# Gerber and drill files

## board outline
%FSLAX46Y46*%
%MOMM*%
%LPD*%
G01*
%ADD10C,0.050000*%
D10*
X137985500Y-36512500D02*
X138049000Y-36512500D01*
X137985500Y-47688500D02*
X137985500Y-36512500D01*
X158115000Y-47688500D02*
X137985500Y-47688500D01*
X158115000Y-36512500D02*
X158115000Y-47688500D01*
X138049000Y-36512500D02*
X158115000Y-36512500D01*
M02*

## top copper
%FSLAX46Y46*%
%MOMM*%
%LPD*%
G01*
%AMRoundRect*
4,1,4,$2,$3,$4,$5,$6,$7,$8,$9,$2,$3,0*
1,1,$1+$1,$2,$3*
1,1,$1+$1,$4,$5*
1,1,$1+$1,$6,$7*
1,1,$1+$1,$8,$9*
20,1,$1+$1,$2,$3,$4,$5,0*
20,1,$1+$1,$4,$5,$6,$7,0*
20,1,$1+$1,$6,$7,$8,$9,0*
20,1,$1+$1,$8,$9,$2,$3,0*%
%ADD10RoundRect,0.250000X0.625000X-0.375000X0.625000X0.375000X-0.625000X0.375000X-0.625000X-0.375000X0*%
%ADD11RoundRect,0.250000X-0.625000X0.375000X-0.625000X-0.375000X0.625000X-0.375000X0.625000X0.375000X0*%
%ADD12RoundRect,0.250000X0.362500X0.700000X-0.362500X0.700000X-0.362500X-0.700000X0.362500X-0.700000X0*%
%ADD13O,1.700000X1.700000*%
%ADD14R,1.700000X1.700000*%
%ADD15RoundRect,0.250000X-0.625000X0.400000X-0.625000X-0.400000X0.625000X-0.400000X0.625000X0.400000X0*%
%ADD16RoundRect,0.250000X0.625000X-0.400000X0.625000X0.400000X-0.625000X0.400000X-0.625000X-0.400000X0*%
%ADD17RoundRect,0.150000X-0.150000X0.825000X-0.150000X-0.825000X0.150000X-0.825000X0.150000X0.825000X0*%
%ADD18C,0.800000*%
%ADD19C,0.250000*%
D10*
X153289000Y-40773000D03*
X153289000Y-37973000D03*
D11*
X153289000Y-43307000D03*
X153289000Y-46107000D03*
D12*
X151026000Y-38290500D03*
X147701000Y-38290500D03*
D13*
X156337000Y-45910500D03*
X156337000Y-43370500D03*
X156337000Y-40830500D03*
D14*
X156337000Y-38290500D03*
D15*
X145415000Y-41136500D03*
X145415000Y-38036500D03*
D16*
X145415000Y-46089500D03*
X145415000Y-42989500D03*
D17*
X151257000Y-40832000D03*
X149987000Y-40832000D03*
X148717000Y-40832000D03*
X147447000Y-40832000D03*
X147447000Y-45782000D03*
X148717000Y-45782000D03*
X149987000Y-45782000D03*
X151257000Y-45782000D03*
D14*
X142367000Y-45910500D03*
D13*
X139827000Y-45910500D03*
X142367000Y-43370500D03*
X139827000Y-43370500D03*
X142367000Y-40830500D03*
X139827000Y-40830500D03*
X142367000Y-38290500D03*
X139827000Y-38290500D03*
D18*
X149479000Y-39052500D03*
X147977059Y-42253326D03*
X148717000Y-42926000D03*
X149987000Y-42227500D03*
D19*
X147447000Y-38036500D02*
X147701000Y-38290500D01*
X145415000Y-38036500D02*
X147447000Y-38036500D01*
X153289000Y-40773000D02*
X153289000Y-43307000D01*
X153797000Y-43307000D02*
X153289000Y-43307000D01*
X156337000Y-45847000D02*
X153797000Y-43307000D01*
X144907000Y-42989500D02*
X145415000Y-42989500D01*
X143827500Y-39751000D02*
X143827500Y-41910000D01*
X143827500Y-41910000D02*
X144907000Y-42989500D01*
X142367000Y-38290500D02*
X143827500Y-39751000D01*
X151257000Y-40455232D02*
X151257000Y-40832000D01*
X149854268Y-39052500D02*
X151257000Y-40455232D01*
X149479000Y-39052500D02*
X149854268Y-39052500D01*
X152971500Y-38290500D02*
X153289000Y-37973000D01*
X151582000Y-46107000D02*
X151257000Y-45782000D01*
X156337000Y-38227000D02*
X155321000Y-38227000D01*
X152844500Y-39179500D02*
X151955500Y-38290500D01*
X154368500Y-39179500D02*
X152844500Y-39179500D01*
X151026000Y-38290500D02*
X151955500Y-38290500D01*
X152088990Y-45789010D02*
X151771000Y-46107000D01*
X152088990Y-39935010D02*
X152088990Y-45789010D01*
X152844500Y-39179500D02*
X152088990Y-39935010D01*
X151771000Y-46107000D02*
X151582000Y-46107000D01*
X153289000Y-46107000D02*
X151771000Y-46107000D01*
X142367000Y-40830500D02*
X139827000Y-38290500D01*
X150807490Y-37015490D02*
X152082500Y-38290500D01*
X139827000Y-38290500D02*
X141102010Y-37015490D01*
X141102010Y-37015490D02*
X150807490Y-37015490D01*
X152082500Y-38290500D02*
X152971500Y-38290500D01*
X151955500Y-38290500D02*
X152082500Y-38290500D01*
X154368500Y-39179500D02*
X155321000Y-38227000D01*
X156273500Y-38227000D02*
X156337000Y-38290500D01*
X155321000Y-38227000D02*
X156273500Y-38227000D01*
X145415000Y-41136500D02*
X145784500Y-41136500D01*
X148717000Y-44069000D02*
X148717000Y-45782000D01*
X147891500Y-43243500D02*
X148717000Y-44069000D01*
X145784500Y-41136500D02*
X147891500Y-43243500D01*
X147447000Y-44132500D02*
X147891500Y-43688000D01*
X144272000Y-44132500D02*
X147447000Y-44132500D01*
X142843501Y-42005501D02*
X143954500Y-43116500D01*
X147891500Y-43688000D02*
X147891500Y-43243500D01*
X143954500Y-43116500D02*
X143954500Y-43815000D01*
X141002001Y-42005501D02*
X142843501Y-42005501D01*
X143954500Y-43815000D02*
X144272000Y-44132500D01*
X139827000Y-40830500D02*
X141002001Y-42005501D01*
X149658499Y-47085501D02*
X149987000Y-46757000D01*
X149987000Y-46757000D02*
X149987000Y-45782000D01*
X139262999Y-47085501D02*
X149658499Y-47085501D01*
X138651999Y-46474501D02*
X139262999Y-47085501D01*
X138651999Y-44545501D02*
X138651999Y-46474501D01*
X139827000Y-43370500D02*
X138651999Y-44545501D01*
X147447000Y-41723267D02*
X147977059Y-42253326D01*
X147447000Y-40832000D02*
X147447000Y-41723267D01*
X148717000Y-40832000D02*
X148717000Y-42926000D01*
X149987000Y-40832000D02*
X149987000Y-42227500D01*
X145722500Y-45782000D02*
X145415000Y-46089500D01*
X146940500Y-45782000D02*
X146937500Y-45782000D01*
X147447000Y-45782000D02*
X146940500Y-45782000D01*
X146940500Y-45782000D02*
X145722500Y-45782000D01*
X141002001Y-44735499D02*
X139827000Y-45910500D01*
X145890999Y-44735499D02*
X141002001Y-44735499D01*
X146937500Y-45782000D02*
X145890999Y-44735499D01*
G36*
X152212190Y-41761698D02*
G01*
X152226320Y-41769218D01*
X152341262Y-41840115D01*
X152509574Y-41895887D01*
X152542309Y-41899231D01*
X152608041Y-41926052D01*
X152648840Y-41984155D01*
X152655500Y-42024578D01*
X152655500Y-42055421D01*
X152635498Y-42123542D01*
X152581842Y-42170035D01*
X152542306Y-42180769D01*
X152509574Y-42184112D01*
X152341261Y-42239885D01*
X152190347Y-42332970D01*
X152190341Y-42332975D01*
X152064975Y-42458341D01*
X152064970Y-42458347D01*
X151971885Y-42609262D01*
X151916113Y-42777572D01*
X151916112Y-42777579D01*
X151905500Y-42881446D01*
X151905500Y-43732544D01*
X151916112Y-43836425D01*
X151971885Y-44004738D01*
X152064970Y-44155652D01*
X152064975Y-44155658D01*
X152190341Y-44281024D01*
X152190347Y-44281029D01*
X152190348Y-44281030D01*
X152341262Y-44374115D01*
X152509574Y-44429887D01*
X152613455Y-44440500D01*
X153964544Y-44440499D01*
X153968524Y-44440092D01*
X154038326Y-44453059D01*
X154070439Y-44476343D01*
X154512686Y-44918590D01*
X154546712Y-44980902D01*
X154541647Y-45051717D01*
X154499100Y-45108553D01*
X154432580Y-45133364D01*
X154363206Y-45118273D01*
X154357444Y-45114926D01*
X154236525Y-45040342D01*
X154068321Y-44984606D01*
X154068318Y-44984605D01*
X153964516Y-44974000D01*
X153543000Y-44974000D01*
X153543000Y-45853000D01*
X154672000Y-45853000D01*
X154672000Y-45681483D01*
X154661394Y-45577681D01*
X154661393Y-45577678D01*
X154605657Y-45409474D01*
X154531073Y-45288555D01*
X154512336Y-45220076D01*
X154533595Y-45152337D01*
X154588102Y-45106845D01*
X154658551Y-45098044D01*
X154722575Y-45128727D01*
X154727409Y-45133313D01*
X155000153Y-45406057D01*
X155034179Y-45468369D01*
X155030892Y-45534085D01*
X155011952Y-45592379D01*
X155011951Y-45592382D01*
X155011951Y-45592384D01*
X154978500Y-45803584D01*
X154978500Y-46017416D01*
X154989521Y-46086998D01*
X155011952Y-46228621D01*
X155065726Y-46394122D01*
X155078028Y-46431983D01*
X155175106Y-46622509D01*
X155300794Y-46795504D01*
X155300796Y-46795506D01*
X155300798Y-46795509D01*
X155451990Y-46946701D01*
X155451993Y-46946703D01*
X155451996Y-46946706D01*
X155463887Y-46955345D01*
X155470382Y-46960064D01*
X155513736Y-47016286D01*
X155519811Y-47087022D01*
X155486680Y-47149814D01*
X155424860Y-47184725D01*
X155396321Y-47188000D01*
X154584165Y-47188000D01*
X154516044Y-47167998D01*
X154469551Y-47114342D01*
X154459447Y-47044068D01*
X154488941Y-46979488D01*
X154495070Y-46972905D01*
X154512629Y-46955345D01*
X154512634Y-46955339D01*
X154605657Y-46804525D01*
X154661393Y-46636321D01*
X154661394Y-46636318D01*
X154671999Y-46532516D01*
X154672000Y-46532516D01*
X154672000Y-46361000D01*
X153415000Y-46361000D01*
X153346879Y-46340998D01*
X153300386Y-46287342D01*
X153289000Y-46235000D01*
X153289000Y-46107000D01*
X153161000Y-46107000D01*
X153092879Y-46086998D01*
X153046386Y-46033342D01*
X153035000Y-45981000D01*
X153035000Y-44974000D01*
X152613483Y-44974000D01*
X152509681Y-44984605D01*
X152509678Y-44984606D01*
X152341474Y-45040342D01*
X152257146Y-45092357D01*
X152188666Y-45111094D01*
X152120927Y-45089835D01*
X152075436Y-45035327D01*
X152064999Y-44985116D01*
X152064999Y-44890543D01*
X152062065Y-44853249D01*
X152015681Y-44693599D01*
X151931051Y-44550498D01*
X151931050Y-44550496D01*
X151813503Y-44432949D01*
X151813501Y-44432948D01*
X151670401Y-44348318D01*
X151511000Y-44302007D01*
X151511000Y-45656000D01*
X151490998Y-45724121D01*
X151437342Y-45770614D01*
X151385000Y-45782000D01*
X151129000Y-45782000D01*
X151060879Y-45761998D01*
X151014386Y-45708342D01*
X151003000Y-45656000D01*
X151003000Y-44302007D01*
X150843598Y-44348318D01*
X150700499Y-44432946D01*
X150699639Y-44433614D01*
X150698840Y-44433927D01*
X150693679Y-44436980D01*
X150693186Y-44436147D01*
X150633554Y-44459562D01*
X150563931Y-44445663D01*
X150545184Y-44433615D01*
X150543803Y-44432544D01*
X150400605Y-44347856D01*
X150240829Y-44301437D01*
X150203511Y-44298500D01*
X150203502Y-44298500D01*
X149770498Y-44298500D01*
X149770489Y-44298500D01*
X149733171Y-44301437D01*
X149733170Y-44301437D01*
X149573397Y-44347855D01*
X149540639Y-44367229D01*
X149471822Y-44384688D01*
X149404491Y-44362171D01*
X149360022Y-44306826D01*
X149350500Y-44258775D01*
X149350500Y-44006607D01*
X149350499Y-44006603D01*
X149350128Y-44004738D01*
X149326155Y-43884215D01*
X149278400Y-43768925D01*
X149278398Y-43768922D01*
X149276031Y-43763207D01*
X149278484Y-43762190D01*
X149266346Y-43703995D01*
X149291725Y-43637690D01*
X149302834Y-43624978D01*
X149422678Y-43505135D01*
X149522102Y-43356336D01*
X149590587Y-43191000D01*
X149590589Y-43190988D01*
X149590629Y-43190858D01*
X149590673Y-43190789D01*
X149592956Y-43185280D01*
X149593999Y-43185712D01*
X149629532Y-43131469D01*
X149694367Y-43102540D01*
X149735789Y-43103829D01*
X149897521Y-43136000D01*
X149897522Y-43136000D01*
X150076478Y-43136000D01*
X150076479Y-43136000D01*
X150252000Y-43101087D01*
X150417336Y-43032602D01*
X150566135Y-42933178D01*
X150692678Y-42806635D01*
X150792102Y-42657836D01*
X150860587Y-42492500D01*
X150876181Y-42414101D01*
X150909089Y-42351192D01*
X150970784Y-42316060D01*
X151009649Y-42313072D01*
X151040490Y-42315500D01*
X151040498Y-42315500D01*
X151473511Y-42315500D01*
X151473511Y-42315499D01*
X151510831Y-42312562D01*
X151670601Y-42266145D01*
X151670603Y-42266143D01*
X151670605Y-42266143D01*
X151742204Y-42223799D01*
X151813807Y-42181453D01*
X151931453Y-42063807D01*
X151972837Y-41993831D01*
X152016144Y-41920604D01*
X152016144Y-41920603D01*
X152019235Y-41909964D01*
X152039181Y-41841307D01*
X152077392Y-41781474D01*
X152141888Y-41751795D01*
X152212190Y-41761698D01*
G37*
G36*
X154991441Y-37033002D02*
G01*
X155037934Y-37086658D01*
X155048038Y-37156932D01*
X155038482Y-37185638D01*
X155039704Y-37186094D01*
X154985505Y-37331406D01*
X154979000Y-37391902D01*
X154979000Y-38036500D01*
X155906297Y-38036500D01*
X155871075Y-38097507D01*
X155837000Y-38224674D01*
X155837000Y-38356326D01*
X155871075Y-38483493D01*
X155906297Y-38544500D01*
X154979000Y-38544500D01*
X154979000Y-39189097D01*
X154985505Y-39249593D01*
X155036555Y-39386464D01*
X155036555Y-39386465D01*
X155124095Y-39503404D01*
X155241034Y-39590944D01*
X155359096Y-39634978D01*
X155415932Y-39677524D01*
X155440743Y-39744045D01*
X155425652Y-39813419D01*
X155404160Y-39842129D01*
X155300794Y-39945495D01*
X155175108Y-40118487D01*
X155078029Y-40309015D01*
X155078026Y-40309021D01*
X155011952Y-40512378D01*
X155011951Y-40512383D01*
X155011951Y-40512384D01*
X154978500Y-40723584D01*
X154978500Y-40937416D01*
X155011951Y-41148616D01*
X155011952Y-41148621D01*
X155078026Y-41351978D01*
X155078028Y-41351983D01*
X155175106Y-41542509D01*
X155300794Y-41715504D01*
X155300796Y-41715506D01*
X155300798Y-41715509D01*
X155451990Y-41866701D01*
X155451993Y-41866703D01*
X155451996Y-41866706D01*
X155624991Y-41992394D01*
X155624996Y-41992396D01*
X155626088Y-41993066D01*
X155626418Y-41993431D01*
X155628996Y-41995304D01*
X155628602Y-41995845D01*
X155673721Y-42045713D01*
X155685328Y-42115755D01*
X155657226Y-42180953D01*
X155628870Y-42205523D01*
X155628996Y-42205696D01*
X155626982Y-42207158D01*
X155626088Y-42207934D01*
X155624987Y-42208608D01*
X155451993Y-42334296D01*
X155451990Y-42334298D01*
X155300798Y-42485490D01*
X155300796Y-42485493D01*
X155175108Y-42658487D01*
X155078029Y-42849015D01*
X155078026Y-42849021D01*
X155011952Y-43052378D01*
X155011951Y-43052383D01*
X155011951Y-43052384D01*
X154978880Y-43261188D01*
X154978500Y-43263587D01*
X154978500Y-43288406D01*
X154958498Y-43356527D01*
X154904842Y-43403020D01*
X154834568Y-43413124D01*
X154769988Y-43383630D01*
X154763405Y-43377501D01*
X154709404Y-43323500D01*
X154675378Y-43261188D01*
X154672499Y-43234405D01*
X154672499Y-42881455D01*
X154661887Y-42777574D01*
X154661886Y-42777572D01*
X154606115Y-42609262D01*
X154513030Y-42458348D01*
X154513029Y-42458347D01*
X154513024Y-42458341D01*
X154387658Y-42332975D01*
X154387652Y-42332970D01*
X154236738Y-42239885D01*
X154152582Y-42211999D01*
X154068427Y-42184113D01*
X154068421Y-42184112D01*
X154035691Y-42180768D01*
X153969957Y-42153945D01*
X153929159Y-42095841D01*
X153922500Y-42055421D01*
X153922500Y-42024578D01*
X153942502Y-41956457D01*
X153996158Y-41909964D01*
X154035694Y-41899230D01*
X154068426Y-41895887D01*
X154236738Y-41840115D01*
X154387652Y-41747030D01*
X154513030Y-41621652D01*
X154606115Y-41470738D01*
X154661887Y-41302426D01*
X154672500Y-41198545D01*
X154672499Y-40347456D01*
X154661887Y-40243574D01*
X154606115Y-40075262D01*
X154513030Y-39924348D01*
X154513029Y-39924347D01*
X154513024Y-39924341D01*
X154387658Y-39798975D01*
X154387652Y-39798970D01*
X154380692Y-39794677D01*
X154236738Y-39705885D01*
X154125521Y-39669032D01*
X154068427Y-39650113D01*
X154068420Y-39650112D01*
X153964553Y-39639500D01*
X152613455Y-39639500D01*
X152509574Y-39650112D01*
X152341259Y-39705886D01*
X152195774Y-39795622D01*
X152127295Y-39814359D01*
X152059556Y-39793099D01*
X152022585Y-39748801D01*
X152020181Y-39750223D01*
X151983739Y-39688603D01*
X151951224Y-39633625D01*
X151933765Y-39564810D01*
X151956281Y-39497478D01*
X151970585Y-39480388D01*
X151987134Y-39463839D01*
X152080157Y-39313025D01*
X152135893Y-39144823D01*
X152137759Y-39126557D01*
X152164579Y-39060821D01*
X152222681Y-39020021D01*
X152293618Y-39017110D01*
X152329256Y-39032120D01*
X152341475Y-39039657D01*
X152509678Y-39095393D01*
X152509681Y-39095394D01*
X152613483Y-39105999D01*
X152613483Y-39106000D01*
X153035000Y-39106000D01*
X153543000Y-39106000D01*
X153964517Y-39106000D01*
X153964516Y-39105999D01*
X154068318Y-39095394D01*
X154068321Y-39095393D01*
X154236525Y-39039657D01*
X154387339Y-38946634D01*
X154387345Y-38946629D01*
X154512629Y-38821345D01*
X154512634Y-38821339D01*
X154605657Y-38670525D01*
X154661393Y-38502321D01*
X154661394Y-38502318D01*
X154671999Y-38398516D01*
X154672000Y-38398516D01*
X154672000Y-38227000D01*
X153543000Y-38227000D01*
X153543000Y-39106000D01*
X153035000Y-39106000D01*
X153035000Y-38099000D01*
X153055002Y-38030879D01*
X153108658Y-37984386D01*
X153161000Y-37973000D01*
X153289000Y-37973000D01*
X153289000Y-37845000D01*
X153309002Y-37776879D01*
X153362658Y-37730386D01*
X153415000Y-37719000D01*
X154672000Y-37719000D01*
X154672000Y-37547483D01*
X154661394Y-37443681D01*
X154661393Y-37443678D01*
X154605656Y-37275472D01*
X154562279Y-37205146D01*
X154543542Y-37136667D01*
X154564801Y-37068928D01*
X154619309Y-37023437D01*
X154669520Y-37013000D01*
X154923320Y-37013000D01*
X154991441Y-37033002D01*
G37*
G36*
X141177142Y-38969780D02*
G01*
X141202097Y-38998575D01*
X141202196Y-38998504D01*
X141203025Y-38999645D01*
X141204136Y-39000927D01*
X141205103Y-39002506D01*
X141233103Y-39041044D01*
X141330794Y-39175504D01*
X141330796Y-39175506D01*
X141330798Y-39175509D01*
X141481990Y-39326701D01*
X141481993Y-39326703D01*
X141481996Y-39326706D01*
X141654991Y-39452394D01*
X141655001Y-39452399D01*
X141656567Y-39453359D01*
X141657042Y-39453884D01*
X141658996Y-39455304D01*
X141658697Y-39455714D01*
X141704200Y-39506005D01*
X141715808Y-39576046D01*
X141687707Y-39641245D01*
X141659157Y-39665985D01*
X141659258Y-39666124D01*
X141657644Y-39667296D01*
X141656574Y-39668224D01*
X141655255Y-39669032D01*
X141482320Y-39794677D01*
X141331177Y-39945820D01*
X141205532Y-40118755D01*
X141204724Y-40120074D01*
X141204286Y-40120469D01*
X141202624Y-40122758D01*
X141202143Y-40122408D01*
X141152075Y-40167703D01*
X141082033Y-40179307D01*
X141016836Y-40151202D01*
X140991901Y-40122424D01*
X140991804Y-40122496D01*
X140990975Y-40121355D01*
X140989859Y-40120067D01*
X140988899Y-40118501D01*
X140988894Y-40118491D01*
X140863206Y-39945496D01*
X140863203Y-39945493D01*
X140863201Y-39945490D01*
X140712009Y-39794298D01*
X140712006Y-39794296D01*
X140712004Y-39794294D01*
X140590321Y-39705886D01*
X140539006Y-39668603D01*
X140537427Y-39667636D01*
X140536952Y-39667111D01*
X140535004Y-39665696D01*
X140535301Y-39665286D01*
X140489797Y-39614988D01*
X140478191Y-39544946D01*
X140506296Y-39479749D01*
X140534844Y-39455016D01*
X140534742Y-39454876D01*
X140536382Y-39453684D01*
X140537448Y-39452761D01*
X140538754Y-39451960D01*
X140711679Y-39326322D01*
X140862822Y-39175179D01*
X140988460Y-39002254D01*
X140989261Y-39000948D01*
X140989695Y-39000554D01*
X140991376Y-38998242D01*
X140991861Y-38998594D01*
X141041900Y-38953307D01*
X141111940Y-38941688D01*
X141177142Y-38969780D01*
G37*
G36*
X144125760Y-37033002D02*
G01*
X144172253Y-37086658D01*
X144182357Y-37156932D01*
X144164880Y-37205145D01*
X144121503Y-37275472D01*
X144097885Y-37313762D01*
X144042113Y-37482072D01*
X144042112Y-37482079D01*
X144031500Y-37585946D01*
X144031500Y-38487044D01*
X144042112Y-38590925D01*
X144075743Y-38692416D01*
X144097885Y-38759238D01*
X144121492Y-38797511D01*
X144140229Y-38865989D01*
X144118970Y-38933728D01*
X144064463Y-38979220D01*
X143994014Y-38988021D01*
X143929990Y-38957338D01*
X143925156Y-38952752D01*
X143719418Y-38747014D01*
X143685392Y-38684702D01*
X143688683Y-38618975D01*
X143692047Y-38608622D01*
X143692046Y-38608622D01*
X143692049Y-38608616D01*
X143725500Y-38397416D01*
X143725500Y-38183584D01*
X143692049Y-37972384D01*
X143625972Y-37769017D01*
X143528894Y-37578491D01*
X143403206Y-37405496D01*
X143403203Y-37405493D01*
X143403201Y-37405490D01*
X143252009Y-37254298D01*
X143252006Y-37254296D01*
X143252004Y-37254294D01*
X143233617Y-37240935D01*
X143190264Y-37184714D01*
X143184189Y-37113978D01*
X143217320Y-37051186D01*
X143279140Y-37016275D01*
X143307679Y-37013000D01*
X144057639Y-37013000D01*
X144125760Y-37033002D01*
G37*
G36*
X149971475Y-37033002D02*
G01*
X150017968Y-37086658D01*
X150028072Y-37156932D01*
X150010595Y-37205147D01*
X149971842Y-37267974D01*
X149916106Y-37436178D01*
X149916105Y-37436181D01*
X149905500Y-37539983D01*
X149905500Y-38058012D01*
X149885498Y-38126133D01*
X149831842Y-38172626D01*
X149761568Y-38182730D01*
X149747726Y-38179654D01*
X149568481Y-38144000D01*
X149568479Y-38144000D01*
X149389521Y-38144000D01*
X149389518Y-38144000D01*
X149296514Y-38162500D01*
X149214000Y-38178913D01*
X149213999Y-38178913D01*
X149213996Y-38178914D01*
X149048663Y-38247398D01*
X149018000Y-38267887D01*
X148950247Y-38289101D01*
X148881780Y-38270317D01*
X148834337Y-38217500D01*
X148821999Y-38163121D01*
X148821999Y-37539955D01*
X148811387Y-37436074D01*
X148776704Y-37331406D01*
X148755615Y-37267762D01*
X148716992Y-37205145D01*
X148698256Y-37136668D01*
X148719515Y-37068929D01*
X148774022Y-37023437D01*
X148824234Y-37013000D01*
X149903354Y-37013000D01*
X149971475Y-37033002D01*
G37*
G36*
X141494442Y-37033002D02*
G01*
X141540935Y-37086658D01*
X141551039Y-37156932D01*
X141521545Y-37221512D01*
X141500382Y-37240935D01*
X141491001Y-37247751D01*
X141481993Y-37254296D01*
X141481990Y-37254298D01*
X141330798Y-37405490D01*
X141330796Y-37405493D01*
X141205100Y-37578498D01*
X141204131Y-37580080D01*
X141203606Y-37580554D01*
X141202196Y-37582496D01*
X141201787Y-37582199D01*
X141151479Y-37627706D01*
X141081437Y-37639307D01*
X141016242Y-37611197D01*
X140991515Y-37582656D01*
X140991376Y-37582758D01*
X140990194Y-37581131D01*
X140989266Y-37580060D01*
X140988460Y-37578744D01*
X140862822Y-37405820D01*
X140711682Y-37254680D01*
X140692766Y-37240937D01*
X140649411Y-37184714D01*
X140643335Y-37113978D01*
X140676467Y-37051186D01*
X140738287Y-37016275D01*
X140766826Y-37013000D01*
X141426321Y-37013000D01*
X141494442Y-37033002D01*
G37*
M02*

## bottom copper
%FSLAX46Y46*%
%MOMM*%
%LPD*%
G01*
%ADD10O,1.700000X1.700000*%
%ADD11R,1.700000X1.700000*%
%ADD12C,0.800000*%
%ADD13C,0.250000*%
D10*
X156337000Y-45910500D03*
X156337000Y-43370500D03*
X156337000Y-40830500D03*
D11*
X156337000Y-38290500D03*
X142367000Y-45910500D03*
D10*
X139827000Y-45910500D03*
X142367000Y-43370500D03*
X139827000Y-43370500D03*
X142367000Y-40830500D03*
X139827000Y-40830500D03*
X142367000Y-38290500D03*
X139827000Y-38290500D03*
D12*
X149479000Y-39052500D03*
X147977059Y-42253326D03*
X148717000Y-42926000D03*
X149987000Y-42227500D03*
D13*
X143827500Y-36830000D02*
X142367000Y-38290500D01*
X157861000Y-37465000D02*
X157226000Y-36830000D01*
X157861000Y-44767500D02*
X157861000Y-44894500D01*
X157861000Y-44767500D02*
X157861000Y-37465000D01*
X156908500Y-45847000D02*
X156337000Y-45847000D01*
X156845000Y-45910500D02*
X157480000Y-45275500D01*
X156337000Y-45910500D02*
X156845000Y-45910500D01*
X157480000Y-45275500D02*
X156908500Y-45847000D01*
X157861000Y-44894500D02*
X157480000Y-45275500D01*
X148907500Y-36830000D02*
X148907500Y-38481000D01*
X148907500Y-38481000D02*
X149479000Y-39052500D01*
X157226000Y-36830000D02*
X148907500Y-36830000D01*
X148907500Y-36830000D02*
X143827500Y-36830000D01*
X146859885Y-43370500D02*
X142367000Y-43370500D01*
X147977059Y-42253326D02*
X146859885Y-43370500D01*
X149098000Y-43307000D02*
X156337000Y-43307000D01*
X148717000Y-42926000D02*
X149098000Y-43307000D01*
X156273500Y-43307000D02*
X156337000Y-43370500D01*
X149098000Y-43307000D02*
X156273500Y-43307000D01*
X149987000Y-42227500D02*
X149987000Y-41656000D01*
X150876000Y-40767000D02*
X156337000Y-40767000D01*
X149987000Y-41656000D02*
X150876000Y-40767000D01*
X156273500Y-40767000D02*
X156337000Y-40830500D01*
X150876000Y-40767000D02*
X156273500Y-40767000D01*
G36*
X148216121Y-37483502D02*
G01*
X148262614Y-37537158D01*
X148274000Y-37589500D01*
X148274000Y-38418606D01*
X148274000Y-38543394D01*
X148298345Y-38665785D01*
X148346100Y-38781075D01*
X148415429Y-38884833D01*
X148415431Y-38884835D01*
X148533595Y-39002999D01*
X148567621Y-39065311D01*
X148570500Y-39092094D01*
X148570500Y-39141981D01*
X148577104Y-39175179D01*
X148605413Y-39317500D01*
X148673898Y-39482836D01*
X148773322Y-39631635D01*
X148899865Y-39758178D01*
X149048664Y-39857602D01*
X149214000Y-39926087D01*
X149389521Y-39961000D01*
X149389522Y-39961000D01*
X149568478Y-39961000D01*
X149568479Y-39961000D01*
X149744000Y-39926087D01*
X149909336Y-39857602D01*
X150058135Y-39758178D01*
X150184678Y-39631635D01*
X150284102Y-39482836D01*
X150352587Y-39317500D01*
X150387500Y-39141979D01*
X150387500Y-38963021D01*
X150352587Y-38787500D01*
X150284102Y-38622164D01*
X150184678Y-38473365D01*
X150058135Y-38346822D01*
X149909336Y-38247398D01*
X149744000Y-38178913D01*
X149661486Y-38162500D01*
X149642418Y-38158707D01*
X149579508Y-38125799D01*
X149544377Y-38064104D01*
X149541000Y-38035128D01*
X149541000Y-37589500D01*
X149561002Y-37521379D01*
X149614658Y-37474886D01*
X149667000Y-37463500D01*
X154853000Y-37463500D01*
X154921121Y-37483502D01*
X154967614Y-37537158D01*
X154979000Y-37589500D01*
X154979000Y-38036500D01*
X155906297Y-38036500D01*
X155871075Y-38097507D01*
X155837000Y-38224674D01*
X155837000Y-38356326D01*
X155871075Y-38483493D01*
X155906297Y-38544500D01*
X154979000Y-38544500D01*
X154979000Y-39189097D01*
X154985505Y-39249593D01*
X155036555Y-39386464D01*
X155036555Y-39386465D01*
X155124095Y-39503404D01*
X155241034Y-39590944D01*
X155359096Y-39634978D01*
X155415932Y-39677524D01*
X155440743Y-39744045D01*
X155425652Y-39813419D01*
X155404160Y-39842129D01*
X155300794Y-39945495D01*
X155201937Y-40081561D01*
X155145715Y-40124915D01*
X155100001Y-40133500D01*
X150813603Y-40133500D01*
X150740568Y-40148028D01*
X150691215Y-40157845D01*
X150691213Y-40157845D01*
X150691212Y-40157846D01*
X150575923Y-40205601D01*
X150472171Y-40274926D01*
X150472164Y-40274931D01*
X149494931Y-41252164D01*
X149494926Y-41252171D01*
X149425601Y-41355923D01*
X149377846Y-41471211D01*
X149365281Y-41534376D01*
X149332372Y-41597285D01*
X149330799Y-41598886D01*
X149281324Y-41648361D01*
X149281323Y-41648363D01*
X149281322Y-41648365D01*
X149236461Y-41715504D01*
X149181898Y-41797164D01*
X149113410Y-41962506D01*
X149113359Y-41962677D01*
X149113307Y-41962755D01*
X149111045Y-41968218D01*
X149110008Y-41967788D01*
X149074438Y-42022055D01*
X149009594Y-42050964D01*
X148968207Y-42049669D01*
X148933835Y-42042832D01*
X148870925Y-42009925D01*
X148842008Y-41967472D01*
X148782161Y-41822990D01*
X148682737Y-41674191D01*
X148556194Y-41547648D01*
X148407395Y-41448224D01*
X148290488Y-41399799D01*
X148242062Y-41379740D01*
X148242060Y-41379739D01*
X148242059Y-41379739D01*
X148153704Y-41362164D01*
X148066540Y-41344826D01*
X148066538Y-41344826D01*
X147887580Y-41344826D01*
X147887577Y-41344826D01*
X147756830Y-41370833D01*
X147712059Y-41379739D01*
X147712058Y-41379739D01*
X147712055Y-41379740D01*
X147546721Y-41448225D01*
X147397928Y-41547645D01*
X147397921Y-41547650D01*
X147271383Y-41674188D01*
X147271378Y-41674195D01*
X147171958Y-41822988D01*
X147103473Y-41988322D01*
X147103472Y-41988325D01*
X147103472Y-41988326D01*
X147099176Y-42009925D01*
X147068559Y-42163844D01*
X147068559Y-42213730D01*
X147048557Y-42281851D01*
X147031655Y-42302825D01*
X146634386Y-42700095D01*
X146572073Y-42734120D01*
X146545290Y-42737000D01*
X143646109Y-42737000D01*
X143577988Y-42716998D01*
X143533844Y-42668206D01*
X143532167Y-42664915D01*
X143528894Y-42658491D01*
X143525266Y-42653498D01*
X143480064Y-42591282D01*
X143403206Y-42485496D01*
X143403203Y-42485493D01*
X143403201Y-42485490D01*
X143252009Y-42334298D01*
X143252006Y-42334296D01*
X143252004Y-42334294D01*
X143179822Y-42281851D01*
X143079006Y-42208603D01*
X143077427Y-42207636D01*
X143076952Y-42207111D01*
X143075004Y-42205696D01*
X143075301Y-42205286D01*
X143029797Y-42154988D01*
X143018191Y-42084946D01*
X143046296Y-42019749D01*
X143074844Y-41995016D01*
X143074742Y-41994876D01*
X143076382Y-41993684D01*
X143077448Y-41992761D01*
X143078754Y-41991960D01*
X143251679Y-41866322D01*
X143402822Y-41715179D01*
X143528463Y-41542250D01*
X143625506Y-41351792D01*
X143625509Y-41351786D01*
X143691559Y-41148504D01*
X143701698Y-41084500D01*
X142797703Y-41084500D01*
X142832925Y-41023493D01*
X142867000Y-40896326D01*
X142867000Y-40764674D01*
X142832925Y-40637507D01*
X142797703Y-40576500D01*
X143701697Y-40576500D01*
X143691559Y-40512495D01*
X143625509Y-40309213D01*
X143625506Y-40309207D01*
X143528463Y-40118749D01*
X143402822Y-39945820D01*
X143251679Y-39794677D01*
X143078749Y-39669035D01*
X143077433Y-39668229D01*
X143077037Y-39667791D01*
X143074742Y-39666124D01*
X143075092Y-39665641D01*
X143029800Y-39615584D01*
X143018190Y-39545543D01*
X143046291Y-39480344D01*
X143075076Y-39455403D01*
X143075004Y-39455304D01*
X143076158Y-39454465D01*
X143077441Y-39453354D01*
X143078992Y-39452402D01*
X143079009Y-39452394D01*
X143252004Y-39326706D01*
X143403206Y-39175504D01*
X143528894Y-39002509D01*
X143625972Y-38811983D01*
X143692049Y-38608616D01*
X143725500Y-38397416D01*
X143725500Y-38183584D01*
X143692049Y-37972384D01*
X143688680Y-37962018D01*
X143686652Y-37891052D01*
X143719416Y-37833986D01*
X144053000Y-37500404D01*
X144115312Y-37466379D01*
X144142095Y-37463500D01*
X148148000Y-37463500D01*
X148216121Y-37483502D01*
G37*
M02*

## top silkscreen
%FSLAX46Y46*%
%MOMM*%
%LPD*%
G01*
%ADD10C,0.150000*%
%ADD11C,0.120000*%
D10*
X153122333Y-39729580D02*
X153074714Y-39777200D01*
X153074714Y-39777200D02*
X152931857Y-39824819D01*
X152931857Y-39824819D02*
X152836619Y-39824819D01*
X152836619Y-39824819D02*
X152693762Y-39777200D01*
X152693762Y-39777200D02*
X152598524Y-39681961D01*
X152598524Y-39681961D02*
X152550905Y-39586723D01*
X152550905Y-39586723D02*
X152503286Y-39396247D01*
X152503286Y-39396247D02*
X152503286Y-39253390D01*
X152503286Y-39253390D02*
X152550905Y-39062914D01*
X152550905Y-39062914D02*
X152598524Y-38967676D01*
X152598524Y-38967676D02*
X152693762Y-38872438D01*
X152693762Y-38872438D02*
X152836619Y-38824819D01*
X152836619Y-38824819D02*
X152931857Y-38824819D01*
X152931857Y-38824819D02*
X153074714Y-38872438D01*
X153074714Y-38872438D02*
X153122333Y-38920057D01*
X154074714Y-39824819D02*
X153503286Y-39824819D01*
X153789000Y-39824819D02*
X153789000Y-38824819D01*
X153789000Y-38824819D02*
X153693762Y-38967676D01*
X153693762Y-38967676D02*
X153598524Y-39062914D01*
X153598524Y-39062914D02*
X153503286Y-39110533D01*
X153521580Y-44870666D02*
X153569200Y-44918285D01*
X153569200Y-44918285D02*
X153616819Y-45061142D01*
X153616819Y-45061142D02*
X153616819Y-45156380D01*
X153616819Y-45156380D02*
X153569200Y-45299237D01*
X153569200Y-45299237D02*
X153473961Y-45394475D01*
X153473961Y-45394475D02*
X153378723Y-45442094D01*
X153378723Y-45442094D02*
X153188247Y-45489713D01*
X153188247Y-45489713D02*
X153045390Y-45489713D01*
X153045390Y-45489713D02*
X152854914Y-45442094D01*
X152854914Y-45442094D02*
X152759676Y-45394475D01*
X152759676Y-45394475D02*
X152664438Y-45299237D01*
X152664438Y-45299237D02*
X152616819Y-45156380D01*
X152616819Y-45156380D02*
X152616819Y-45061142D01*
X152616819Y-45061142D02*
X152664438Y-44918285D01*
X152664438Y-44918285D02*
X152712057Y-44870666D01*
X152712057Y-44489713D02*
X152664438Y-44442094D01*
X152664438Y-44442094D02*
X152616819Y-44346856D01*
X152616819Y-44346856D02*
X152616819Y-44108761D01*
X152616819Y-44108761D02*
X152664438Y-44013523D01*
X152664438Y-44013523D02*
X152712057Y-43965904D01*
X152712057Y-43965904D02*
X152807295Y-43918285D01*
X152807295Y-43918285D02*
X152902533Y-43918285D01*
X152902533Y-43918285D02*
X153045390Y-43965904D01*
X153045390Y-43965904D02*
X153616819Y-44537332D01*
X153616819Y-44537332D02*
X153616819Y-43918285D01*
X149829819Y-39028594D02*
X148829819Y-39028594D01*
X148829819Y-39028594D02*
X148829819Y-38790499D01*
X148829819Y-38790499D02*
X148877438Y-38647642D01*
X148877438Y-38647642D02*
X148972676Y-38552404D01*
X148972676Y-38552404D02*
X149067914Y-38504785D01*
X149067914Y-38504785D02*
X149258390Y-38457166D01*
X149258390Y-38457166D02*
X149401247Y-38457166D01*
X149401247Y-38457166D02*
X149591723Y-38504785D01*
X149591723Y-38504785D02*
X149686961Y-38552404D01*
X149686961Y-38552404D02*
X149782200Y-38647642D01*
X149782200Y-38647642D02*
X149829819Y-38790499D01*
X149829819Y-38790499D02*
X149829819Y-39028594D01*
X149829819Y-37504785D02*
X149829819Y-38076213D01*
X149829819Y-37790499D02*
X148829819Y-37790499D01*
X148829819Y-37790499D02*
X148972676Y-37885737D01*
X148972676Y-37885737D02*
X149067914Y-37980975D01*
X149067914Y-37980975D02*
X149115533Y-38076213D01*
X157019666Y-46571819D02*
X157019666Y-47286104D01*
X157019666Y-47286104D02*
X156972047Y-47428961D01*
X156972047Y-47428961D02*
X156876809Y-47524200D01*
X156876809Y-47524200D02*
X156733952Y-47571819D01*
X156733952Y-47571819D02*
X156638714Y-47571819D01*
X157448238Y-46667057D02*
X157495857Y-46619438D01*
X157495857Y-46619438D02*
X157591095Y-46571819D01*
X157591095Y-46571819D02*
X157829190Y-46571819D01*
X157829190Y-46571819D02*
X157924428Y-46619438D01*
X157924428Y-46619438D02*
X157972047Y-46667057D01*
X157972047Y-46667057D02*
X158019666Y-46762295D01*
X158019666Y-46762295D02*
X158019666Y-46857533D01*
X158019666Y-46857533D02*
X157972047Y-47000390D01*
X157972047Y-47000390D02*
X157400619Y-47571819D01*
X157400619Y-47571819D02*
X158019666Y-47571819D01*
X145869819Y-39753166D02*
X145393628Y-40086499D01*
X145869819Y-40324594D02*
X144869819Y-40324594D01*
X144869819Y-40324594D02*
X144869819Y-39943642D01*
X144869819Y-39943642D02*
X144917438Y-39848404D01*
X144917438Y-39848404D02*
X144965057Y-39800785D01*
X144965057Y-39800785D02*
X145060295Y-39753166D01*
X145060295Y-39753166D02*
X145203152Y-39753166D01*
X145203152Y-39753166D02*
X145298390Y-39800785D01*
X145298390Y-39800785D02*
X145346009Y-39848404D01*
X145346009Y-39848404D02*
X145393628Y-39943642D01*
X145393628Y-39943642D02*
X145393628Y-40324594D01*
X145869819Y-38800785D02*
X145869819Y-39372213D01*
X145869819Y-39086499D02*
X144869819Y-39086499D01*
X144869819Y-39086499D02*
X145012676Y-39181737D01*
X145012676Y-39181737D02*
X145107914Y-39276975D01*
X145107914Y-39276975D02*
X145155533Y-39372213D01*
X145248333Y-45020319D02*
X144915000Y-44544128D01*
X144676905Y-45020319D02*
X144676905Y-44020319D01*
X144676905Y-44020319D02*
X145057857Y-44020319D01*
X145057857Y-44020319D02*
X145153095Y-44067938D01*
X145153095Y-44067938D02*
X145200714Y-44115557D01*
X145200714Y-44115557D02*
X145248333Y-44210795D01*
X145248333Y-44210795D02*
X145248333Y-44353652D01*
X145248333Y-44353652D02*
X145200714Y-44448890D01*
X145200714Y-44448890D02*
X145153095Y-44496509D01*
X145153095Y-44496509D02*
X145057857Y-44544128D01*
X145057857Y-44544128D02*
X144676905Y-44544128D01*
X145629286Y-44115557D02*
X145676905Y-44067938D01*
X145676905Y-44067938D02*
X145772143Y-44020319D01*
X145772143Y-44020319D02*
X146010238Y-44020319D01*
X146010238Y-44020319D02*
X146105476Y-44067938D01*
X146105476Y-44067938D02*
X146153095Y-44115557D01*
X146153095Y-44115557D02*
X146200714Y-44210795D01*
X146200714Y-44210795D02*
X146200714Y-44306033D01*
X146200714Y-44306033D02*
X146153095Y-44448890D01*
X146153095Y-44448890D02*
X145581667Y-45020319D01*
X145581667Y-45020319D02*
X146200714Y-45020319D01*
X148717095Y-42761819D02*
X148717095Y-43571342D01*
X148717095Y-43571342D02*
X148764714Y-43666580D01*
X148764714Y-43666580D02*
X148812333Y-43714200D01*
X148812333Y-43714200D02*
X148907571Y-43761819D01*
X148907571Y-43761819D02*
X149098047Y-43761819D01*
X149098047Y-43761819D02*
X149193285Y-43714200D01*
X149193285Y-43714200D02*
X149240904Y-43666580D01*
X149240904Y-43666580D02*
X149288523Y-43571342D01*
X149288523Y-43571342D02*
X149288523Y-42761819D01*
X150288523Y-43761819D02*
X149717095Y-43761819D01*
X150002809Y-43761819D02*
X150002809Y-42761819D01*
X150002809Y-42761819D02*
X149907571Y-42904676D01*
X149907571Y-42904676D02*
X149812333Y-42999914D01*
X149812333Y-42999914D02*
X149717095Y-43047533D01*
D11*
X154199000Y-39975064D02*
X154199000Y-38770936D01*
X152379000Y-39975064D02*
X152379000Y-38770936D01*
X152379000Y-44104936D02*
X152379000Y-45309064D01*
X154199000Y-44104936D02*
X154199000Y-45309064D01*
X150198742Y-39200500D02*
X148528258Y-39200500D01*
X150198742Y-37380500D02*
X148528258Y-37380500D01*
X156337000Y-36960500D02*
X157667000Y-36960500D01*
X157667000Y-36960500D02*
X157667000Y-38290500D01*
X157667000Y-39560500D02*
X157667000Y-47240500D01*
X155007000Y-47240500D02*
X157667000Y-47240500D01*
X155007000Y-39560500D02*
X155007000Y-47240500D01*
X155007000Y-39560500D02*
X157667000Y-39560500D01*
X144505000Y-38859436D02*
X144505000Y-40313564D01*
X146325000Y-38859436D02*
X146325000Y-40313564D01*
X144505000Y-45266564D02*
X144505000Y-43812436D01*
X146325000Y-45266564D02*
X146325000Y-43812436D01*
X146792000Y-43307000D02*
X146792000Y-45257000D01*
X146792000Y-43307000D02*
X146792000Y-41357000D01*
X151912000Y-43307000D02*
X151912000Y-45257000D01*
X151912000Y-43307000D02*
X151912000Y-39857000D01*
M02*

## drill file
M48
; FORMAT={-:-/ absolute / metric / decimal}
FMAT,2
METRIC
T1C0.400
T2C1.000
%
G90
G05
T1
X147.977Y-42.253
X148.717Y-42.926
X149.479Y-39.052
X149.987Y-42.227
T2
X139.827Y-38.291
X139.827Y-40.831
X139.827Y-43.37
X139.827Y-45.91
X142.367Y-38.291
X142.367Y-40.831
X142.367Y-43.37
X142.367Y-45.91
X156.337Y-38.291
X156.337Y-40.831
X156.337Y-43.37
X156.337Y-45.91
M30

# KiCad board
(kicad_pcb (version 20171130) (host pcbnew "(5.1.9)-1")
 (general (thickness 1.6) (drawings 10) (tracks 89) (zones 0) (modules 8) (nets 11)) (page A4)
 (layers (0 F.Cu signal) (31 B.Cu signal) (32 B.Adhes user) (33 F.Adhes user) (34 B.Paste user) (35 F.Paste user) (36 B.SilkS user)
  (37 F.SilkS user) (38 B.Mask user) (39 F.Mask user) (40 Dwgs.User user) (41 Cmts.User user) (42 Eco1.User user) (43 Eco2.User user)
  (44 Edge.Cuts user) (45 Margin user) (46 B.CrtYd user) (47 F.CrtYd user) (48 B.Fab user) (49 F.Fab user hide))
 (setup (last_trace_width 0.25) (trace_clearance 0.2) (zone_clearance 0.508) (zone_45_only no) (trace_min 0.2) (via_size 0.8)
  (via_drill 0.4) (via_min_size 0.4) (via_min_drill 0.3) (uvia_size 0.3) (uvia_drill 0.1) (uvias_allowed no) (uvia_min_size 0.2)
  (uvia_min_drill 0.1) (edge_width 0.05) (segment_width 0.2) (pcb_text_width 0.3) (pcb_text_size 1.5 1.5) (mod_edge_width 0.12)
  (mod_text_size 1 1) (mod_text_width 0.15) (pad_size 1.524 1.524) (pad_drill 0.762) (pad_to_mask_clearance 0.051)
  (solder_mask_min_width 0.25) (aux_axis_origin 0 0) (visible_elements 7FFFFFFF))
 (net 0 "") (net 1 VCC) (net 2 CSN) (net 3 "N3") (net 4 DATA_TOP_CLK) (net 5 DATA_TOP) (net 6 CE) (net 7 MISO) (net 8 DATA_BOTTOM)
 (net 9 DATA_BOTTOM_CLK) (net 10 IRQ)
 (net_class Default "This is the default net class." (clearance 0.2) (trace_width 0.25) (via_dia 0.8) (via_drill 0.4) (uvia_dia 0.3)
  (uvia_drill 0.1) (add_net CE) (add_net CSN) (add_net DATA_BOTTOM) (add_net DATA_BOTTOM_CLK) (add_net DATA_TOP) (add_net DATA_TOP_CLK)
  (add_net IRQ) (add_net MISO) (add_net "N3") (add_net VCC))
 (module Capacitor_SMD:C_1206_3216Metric (layer F.Cu) (at 153.289 39.373 90)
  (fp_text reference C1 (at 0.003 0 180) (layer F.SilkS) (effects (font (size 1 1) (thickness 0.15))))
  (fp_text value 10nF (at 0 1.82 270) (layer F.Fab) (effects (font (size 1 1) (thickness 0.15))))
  (fp_line (start -0.602064 0.91) (end 0.602064 0.91) (layer F.SilkS) (width 0.12))
  (fp_line (start -0.602064 -0.91) (end 0.602064 -0.91) (layer F.SilkS) (width 0.12))
  (pad 1 smd roundrect (at -1.4 0 90) (size 1.25 1.75) (layers F.Cu F.Paste F.Mask) (roundrect_rratio 0.2) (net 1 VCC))
  (pad 2 smd roundrect (at 1.4 0 90) (size 1.25 1.75) (layers F.Cu F.Paste F.Mask) (roundrect_rratio 0.2) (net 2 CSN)))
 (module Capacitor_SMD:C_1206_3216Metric (layer F.Cu) (at 153.289 44.707 270)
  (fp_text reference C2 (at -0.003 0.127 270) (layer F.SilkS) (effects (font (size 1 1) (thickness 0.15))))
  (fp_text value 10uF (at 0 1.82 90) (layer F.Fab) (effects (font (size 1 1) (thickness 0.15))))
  (fp_line (start -0.602064 0.91) (end 0.602064 0.91) (layer F.SilkS) (width 0.12))
  (fp_line (start -0.602064 -0.91) (end 0.602064 -0.91) (layer F.SilkS) (width 0.12))
  (pad 1 smd roundrect (at -1.4 0 270) (size 1.25 1.75) (layers F.Cu F.Paste F.Mask) (roundrect_rratio 0.2) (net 1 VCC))
  (pad 2 smd roundrect (at 1.4 0 270) (size 1.25 1.75) (layers F.Cu F.Paste F.Mask) (roundrect_rratio 0.2) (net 2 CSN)))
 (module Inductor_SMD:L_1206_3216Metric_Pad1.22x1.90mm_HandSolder (layer F.Cu) (at 149.3635 38.2905 180)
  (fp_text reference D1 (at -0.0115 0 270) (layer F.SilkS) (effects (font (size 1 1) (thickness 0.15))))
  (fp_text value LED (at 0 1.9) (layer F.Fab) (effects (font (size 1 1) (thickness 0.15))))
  (fp_line (start -0.835242 -0.91) (end 0.835242 -0.91) (layer F.SilkS) (width 0.12))
  (fp_line (start -0.835242 0.91) (end 0.835242 0.91) (layer F.SilkS) (width 0.12))
  (pad 1 smd roundrect (at -1.6625 0 180) (size 1.225 1.9) (layers F.Cu F.Paste F.Mask) (roundrect_rratio 0.204082) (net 2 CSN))
  (pad 2 smd roundrect (at 1.6625 0 180) (size 1.225 1.9) (layers F.Cu F.Paste F.Mask) (roundrect_rratio 0.204082) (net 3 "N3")))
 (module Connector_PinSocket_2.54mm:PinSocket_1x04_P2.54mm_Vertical (layer F.Cu) (at 156.337 38.2905)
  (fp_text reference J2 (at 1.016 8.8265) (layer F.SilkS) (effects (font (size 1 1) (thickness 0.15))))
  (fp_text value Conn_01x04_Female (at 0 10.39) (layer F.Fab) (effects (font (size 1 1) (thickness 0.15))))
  (fp_line (start 0 -1.33) (end 1.33 -1.33) (layer F.SilkS) (width 0.12))
  (fp_line (start 1.33 -1.33) (end 1.33 0) (layer F.SilkS) (width 0.12))
  (fp_line (start 1.33 1.27) (end 1.33 8.95) (layer F.SilkS) (width 0.12))
  (fp_line (start -1.33 8.95) (end 1.33 8.95) (layer F.SilkS) (width 0.12))
  (fp_line (start -1.33 1.27) (end -1.33 8.95) (layer F.SilkS) (width 0.12))
  (fp_line (start -1.33 1.27) (end 1.33 1.27) (layer F.SilkS) (width 0.12))
  (pad 4 thru_hole oval (at 0 7.62) (size 1.7 1.7) (drill 1) (layers *.Cu *.Mask) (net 1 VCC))
  (pad 3 thru_hole oval (at 0 5.08) (size 1.7 1.7) (drill 1) (layers *.Cu *.Mask) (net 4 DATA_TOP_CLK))
  (pad 2 thru_hole oval (at 0 2.54) (size 1.7 1.7) (drill 1) (layers *.Cu *.Mask) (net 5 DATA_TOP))
  (pad 1 thru_hole rect (at 0 0) (size 1.7 1.7) (drill 1) (layers *.Cu *.Mask) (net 2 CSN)))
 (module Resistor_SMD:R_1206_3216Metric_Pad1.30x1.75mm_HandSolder (layer F.Cu) (at 145.415 39.5865 270)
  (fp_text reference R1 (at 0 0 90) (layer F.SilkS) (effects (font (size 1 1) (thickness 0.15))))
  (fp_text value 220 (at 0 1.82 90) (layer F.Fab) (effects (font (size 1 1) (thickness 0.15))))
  (fp_line (start -0.727064 0.91) (end 0.727064 0.91) (layer F.SilkS) (width 0.12))
  (fp_line (start -0.727064 -0.91) (end 0.727064 -0.91) (layer F.SilkS) (width 0.12))
  (pad 2 smd roundrect (at 1.55 0 270) (size 1.3 1.75) (layers F.Cu F.Paste F.Mask) (roundrect_rratio 0.192308) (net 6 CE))
  (pad 1 smd roundrect (at -1.55 0 270) (size 1.3 1.75) (layers F.Cu F.Paste F.Mask) (roundrect_rratio 0.192308) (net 3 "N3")))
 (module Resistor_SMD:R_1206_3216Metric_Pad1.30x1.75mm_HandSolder (layer F.Cu) (at 145.415 44.5395 90)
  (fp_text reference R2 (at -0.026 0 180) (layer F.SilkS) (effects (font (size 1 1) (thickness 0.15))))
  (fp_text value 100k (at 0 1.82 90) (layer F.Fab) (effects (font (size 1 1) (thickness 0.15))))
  (fp_line (start -0.727064 -0.91) (end 0.727064 -0.91) (layer F.SilkS) (width 0.12))
  (fp_line (start -0.727064 0.91) (end 0.727064 0.91) (layer F.SilkS) (width 0.12))
  (pad 1 smd roundrect (at -1.55 0 90) (size 1.3 1.75) (layers F.Cu F.Paste F.Mask) (roundrect_rratio 0.192308) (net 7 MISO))
  (pad 2 smd roundrect (at 1.55 0 90) (size 1.3 1.75) (layers F.Cu F.Paste F.Mask) (roundrect_rratio 0.192308) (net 1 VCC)))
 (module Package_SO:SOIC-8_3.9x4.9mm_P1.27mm (layer F.Cu) (at 149.352 43.307 270)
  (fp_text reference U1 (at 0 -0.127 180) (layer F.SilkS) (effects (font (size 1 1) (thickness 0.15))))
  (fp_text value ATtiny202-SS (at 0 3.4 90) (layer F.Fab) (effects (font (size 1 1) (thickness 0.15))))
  (fp_line (start 0 2.56) (end 1.95 2.56) (layer F.SilkS) (width 0.12))
  (fp_line (start 0 2.56) (end -1.95 2.56) (layer F.SilkS) (width 0.12))
  (fp_line (start 0 -2.56) (end 1.95 -2.56) (layer F.SilkS) (width 0.12))
  (fp_line (start 0 -2.56) (end -3.45 -2.56) (layer F.SilkS) (width 0.12))
  (pad 1 smd roundrect (at -2.475 -1.905 270) (size 1.95 0.6) (layers F.Cu F.Paste F.Mask) (roundrect_rratio 0.25) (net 1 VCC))
  (pad 2 smd roundrect (at -2.475 -0.635 270) (size 1.95 0.6) (layers F.Cu F.Paste F.Mask) (roundrect_rratio 0.25) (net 5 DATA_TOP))
  (pad 3 smd roundrect (at -2.475 0.635 270) (size 1.95 0.6) (layers F.Cu F.Paste F.Mask) (roundrect_rratio 0.25) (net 4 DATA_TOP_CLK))
  (pad 4 smd roundrect (at -2.475 1.905 270) (size 1.95 0.6) (layers F.Cu F.Paste F.Mask) (roundrect_rratio 0.25) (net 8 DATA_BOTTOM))
  (pad 5 smd roundrect (at 2.475 1.905 270) (size 1.95 0.6) (layers F.Cu F.Paste F.Mask) (roundrect_rratio 0.25) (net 7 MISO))
  (pad 6 smd roundrect (at 2.475 0.635 270) (size 1.95 0.6) (layers F.Cu F.Paste F.Mask) (roundrect_rratio 0.25) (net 6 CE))
  (pad 7 smd roundrect (at 2.475 -0.635 270) (size 1.95 0.6) (layers F.Cu F.Paste F.Mask) (roundrect_rratio 0.25) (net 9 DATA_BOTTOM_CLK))
  (pad 8 smd roundrect (at 2.475 -1.905 270) (size 1.95 0.6) (layers F.Cu F.Paste F.Mask) (roundrect_rratio 0.25) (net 2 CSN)))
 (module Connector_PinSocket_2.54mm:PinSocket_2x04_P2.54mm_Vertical (layer B.Cu) (at 142.367 45.9105)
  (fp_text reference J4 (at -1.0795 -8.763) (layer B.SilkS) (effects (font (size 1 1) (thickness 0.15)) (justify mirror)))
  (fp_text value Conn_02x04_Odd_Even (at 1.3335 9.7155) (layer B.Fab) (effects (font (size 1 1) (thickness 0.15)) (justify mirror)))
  (pad 1 thru_hole rect (at 0 0) (size 1.7 1.7) (drill 1) (layers *.Cu *.Mask) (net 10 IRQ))
  (pad 2 thru_hole oval (at -2.54 0) (size 1.7 1.7) (drill 1) (layers *.Cu *.Mask) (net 7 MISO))
  (pad 3 thru_hole oval (at 0 -2.54) (size 1.7 1.7) (drill 1) (layers *.Cu *.Mask) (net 8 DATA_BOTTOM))
  (pad 4 thru_hole oval (at -2.54 -2.54) (size 1.7 1.7) (drill 1) (layers *.Cu *.Mask) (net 9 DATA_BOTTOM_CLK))
  (pad 5 thru_hole oval (at 0 -5.08) (size 1.7 1.7) (drill 1) (layers *.Cu *.Mask) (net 2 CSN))
  (pad 6 thru_hole oval (at -2.54 -5.08) (size 1.7 1.7) (drill 1) (layers *.Cu *.Mask) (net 6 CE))
  (pad 7 thru_hole oval (at 0 -7.62) (size 1.7 1.7) (drill 1) (layers *.Cu *.Mask) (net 1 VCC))
  (pad 8 thru_hole oval (at -2.54 -7.62) (size 1.7 1.7) (drill 1) (layers *.Cu *.Mask) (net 2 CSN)))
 (gr_line (start 137.9855 36.5125) (end 138.049 36.5125) (layer Edge.Cuts) (width 0.05))
 (gr_line (start 137.9855 47.6885) (end 137.9855 36.5125) (layer Edge.Cuts) (width 0.05))
 (gr_line (start 158.115 47.6885) (end 137.9855 47.6885) (layer Edge.Cuts) (width 0.05))
 (gr_line (start 158.115 36.5125) (end 158.115 47.6885) (layer Edge.Cuts) (width 0.05))
 (gr_line (start 138.049 36.5125) (end 158.115 36.5125) (layer Edge.Cuts) (width 0.05))
 (segment (start 147.447 38.0365) (end 147.701 38.2905) (width 0.25) (layer F.Cu) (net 3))
 (segment (start 145.415 38.0365) (end 147.447 38.0365) (width 0.25) (layer F.Cu) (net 3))
 (segment (start 153.289 40.773) (end 153.289 43.307) (width 0.25) (layer F.Cu) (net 1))
 (segment (start 153.797 43.307) (end 153.289 43.307) (width 0.25) (layer F.Cu) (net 1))
 (segment (start 156.337 45.847) (end 153.797 43.307) (width 0.25) (layer F.Cu) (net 1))
 (segment (start 144.907 42.9895) (end 145.415 42.9895) (width 0.25) (layer F.Cu) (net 1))
 (segment (start 143.8275 39.751) (end 143.8275 41.91) (width 0.25) (layer F.Cu) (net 1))
 (segment (start 143.8275 41.91) (end 144.907 42.9895) (width 0.25) (layer F.Cu) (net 1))
 (segment (start 142.367 38.2905) (end 143.8275 39.751) (width 0.25) (layer F.Cu) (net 1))
 (segment (start 143.8275 36.83) (end 142.367 38.2905) (width 0.25) (layer B.Cu) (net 1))
 (segment (start 157.861 37.465) (end 157.226 36.83) (width 0.25) (layer B.Cu) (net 1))
 (segment (start 157.861 44.7675) (end 157.861 44.8945) (width 0.25) (layer B.Cu) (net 1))
 (segment (start 157.861 44.7675) (end 157.861 37.465) (width 0.25) (layer B.Cu) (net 1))
 (segment (start 156.9085 45.847) (end 156.337 45.847) (width 0.25) (layer B.Cu) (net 1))
 (segment (start 156.845 45.9105) (end 157.48 45.2755) (width 0.25) (layer B.Cu) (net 1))
 (segment (start 156.337 45.9105) (end 156.845 45.9105) (width 0.25) (layer B.Cu) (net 1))
 (segment (start 157.48 45.2755) (end 156.9085 45.847) (width 0.25) (layer B.Cu) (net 1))
 (segment (start 157.861 44.8945) (end 157.48 45.2755) (width 0.25) (layer B.Cu) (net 1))
 (via (at 149.479 39.0525) (size 0.8) (drill 0.4) (layers F.Cu B.Cu) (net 1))
 (segment (start 148.9075 36.83) (end 148.9075 38.481) (width 0.25) (layer B.Cu) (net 1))
 (segment (start 148.9075 38.481) (end 149.479 39.0525) (width 0.25) (layer B.Cu) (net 1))
 (segment (start 157.226 36.83) (end 148.9075 36.83) (width 0.25) (layer B.Cu) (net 1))
 (segment (start 148.9075 36.83) (end 143.8275 36.83) (width 0.25) (layer B.Cu) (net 1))
 (segment (start 151.257 40.455232) (end 151.257 40.832) (width 0.25) (layer F.Cu) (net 1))
 (segment (start 149.854268 39.0525) (end 151.257 40.455232) (width 0.25) (layer F.Cu) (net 1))
 (segment (start 149.479 39.0525) (end 149.854268 39.0525) (width 0.25) (layer F.Cu) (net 1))
 (segment (start 152.9715 38.2905) (end 153.289 37.973) (width 0.25) (layer F.Cu) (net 2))
 (segment (start 151.582 46.107) (end 151.257 45.782) (width 0.25) (layer F.Cu) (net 2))
 (segment (start 156.337 38.227) (end 155.321 38.227) (width 0.25) (layer F.Cu) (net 2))
 (segment (start 152.8445 39.1795) (end 151.9555 38.2905) (width 0.25) (layer F.Cu) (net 2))
 (segment (start 154.3685 39.1795) (end 152.8445 39.1795) (width 0.25) (layer F.Cu) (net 2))
 (segment (start 151.026 38.2905) (end 151.9555 38.2905) (width 0.25) (layer F.Cu) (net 2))
 (segment (start 152.08899 45.78901) (end 151.771 46.107) (width 0.25) (layer F.Cu) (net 2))
 (segment (start 152.08899 39.93501) (end 152.08899 45.78901) (width 0.25) (layer F.Cu) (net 2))
 (segment (start 152.8445 39.1795) (end 152.08899 39.93501) (width 0.25) (layer F.Cu) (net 2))
 (segment (start 151.771 46.107) (end 151.582 46.107) (width 0.25) (layer F.Cu) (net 2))
 (segment (start 153.289 46.107) (end 151.771 46.107) (width 0.25) (layer F.Cu) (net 2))
 (segment (start 142.367 40.8305) (end 139.827 38.2905) (width 0.25) (layer F.Cu) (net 2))
 (segment (start 150.80749 37.01549) (end 152.0825 38.2905) (width 0.25) (layer F.Cu) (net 2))
 (segment (start 139.827 38.2905) (end 141.10201 37.01549) (width 0.25) (layer F.Cu) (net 2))
 (segment (start 141.10201 37.01549) (end 150.80749 37.01549) (width 0.25) (layer F.Cu) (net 2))
 (segment (start 152.0825 38.2905) (end 152.9715 38.2905) (width 0.25) (layer F.Cu) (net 2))
 (segment (start 151.9555 38.2905) (end 152.0825 38.2905) (width 0.25) (layer F.Cu) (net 2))
 (segment (start 154.3685 39.1795) (end 155.321 38.227) (width 0.25) (layer F.Cu) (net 2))
 (segment (start 156.2735 38.227) (end 156.337 38.2905) (width 0.25) (layer F.Cu) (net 2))
 (segment (start 155.321 38.227) (end 156.2735 38.227) (width 0.25) (layer F.Cu) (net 2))
 (segment (start 145.415 41.1365) (end 145.7845 41.1365) (width 0.25) (layer F.Cu) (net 6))
 (segment (start 148.717 44.069) (end 148.717 45.782) (width 0.25) (layer F.Cu) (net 6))
 (segment (start 147.8915 43.2435) (end 148.717 44.069) (width 0.25) (layer F.Cu) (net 6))
 (segment (start 145.7845 41.1365) (end 147.8915 43.2435) (width 0.25) (layer F.Cu) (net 6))
 (segment (start 147.447 44.1325) (end 147.8915 43.688) (width 0.25) (layer F.Cu) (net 6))
 (segment (start 144.272 44.1325) (end 147.447 44.1325) (width 0.25) (layer F.Cu) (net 6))
 (segment (start 142.843501 42.005501) (end 143.9545 43.1165) (width 0.25) (layer F.Cu) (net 6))
 (segment (start 147.8915 43.688) (end 147.8915 43.2435) (width 0.25) (layer F.Cu) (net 6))
 (segment (start 143.9545 43.1165) (end 143.9545 43.815) (width 0.25) (layer F.Cu) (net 6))
 (segment (start 141.002001 42.005501) (end 142.843501 42.005501) (width 0.25) (layer F.Cu) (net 6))
 (segment (start 143.9545 43.815) (end 144.272 44.1325) (width 0.25) (layer F.Cu) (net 6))
 (segment (start 139.827 40.8305) (end 141.002001 42.005501) (width 0.25) (layer F.Cu) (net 6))
 (segment (start 149.658499 47.085501) (end 149.987 46.757) (width 0.25) (layer F.Cu) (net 9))
 (segment (start 149.987 46.757) (end 149.987 45.782) (width 0.25) (layer F.Cu) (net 9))
 (segment (start 139.262999 47.085501) (end 149.658499 47.085501) (width 0.25) (layer F.Cu) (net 9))
 (segment (start 138.651999 46.474501) (end 139.262999 47.085501) (width 0.25) (layer F.Cu) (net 9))
 (segment (start 138.651999 44.545501) (end 138.651999 46.474501) (width 0.25) (layer F.Cu) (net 9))
 (segment (start 139.827 43.3705) (end 138.651999 44.545501) (width 0.25) (layer F.Cu) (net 9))
 (via (at 147.977059 42.253326) (size 0.8) (drill 0.4) (layers F.Cu B.Cu) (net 8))
 (segment (start 147.447 41.723267) (end 147.977059 42.253326) (width 0.25) (layer F.Cu) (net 8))
 (segment (start 147.447 40.832) (end 147.447 41.723267) (width 0.25) (layer F.Cu) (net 8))
 (segment (start 146.859885 43.3705) (end 142.367 43.3705) (width 0.25) (layer B.Cu) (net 8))
 (segment (start 147.977059 42.253326) (end 146.859885 43.3705) (width 0.25) (layer B.Cu) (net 8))
 (via (at 148.717 42.926) (size 0.8) (drill 0.4) (layers F.Cu B.Cu) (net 4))
 (segment (start 148.717 40.832) (end 148.717 42.926) (width 0.25) (layer F.Cu) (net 4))
 (segment (start 149.098 43.307) (end 156.337 43.307) (width 0.25) (layer B.Cu) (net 4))
 (segment (start 148.717 42.926) (end 149.098 43.307) (width 0.25) (layer B.Cu) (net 4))
 (segment (start 156.2735 43.307) (end 156.337 43.3705) (width 0.25) (layer B.Cu) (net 4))
 (segment (start 149.098 43.307) (end 156.2735 43.307) (width 0.25) (layer B.Cu) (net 4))
 (via (at 149.987 42.2275) (size 0.8) (drill 0.4) (layers F.Cu B.Cu) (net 5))
 (segment (start 149.987 40.832) (end 149.987 42.2275) (width 0.25) (layer F.Cu) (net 5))
 (segment (start 149.987 42.2275) (end 149.987 41.656) (width 0.25) (layer B.Cu) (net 5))
 (segment (start 150.876 40.767) (end 156.337 40.767) (width 0.25) (layer B.Cu) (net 5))
 (segment (start 149.987 41.656) (end 150.876 40.767) (width 0.25) (layer B.Cu) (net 5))
 (segment (start 156.2735 40.767) (end 156.337 40.8305) (width 0.25) (layer B.Cu) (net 5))
 (segment (start 150.876 40.767) (end 156.2735 40.767) (width 0.25) (layer B.Cu) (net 5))
 (segment (start 145.7225 45.782) (end 145.415 46.0895) (width 0.25) (layer F.Cu) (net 7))
 (segment (start 146.9405 45.782) (end 146.9375 45.782) (width 0.25) (layer F.Cu) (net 7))
 (segment (start 147.447 45.782) (end 146.9405 45.782) (width 0.25) (layer F.Cu) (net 7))
 (segment (start 146.9405 45.782) (end 145.7225 45.782) (width 0.25) (layer F.Cu) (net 7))
 (segment (start 141.002001 44.735499) (end 139.827 45.9105) (width 0.25) (layer F.Cu) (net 7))
 (segment (start 145.890999 44.735499) (end 141.002001 44.735499) (width 0.25) (layer F.Cu) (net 7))
 (segment (start 146.9375 45.782) (end 145.890999 44.735499) (width 0.25) (layer F.Cu) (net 7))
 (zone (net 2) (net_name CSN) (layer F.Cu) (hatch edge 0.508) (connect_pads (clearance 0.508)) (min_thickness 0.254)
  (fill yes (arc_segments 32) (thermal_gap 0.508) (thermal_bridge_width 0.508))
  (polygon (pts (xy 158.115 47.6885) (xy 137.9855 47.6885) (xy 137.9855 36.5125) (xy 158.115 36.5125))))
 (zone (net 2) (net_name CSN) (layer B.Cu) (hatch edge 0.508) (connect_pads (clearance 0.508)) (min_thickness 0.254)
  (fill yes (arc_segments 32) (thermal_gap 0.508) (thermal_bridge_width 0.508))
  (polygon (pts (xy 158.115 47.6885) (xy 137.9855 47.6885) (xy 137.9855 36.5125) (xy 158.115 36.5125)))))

